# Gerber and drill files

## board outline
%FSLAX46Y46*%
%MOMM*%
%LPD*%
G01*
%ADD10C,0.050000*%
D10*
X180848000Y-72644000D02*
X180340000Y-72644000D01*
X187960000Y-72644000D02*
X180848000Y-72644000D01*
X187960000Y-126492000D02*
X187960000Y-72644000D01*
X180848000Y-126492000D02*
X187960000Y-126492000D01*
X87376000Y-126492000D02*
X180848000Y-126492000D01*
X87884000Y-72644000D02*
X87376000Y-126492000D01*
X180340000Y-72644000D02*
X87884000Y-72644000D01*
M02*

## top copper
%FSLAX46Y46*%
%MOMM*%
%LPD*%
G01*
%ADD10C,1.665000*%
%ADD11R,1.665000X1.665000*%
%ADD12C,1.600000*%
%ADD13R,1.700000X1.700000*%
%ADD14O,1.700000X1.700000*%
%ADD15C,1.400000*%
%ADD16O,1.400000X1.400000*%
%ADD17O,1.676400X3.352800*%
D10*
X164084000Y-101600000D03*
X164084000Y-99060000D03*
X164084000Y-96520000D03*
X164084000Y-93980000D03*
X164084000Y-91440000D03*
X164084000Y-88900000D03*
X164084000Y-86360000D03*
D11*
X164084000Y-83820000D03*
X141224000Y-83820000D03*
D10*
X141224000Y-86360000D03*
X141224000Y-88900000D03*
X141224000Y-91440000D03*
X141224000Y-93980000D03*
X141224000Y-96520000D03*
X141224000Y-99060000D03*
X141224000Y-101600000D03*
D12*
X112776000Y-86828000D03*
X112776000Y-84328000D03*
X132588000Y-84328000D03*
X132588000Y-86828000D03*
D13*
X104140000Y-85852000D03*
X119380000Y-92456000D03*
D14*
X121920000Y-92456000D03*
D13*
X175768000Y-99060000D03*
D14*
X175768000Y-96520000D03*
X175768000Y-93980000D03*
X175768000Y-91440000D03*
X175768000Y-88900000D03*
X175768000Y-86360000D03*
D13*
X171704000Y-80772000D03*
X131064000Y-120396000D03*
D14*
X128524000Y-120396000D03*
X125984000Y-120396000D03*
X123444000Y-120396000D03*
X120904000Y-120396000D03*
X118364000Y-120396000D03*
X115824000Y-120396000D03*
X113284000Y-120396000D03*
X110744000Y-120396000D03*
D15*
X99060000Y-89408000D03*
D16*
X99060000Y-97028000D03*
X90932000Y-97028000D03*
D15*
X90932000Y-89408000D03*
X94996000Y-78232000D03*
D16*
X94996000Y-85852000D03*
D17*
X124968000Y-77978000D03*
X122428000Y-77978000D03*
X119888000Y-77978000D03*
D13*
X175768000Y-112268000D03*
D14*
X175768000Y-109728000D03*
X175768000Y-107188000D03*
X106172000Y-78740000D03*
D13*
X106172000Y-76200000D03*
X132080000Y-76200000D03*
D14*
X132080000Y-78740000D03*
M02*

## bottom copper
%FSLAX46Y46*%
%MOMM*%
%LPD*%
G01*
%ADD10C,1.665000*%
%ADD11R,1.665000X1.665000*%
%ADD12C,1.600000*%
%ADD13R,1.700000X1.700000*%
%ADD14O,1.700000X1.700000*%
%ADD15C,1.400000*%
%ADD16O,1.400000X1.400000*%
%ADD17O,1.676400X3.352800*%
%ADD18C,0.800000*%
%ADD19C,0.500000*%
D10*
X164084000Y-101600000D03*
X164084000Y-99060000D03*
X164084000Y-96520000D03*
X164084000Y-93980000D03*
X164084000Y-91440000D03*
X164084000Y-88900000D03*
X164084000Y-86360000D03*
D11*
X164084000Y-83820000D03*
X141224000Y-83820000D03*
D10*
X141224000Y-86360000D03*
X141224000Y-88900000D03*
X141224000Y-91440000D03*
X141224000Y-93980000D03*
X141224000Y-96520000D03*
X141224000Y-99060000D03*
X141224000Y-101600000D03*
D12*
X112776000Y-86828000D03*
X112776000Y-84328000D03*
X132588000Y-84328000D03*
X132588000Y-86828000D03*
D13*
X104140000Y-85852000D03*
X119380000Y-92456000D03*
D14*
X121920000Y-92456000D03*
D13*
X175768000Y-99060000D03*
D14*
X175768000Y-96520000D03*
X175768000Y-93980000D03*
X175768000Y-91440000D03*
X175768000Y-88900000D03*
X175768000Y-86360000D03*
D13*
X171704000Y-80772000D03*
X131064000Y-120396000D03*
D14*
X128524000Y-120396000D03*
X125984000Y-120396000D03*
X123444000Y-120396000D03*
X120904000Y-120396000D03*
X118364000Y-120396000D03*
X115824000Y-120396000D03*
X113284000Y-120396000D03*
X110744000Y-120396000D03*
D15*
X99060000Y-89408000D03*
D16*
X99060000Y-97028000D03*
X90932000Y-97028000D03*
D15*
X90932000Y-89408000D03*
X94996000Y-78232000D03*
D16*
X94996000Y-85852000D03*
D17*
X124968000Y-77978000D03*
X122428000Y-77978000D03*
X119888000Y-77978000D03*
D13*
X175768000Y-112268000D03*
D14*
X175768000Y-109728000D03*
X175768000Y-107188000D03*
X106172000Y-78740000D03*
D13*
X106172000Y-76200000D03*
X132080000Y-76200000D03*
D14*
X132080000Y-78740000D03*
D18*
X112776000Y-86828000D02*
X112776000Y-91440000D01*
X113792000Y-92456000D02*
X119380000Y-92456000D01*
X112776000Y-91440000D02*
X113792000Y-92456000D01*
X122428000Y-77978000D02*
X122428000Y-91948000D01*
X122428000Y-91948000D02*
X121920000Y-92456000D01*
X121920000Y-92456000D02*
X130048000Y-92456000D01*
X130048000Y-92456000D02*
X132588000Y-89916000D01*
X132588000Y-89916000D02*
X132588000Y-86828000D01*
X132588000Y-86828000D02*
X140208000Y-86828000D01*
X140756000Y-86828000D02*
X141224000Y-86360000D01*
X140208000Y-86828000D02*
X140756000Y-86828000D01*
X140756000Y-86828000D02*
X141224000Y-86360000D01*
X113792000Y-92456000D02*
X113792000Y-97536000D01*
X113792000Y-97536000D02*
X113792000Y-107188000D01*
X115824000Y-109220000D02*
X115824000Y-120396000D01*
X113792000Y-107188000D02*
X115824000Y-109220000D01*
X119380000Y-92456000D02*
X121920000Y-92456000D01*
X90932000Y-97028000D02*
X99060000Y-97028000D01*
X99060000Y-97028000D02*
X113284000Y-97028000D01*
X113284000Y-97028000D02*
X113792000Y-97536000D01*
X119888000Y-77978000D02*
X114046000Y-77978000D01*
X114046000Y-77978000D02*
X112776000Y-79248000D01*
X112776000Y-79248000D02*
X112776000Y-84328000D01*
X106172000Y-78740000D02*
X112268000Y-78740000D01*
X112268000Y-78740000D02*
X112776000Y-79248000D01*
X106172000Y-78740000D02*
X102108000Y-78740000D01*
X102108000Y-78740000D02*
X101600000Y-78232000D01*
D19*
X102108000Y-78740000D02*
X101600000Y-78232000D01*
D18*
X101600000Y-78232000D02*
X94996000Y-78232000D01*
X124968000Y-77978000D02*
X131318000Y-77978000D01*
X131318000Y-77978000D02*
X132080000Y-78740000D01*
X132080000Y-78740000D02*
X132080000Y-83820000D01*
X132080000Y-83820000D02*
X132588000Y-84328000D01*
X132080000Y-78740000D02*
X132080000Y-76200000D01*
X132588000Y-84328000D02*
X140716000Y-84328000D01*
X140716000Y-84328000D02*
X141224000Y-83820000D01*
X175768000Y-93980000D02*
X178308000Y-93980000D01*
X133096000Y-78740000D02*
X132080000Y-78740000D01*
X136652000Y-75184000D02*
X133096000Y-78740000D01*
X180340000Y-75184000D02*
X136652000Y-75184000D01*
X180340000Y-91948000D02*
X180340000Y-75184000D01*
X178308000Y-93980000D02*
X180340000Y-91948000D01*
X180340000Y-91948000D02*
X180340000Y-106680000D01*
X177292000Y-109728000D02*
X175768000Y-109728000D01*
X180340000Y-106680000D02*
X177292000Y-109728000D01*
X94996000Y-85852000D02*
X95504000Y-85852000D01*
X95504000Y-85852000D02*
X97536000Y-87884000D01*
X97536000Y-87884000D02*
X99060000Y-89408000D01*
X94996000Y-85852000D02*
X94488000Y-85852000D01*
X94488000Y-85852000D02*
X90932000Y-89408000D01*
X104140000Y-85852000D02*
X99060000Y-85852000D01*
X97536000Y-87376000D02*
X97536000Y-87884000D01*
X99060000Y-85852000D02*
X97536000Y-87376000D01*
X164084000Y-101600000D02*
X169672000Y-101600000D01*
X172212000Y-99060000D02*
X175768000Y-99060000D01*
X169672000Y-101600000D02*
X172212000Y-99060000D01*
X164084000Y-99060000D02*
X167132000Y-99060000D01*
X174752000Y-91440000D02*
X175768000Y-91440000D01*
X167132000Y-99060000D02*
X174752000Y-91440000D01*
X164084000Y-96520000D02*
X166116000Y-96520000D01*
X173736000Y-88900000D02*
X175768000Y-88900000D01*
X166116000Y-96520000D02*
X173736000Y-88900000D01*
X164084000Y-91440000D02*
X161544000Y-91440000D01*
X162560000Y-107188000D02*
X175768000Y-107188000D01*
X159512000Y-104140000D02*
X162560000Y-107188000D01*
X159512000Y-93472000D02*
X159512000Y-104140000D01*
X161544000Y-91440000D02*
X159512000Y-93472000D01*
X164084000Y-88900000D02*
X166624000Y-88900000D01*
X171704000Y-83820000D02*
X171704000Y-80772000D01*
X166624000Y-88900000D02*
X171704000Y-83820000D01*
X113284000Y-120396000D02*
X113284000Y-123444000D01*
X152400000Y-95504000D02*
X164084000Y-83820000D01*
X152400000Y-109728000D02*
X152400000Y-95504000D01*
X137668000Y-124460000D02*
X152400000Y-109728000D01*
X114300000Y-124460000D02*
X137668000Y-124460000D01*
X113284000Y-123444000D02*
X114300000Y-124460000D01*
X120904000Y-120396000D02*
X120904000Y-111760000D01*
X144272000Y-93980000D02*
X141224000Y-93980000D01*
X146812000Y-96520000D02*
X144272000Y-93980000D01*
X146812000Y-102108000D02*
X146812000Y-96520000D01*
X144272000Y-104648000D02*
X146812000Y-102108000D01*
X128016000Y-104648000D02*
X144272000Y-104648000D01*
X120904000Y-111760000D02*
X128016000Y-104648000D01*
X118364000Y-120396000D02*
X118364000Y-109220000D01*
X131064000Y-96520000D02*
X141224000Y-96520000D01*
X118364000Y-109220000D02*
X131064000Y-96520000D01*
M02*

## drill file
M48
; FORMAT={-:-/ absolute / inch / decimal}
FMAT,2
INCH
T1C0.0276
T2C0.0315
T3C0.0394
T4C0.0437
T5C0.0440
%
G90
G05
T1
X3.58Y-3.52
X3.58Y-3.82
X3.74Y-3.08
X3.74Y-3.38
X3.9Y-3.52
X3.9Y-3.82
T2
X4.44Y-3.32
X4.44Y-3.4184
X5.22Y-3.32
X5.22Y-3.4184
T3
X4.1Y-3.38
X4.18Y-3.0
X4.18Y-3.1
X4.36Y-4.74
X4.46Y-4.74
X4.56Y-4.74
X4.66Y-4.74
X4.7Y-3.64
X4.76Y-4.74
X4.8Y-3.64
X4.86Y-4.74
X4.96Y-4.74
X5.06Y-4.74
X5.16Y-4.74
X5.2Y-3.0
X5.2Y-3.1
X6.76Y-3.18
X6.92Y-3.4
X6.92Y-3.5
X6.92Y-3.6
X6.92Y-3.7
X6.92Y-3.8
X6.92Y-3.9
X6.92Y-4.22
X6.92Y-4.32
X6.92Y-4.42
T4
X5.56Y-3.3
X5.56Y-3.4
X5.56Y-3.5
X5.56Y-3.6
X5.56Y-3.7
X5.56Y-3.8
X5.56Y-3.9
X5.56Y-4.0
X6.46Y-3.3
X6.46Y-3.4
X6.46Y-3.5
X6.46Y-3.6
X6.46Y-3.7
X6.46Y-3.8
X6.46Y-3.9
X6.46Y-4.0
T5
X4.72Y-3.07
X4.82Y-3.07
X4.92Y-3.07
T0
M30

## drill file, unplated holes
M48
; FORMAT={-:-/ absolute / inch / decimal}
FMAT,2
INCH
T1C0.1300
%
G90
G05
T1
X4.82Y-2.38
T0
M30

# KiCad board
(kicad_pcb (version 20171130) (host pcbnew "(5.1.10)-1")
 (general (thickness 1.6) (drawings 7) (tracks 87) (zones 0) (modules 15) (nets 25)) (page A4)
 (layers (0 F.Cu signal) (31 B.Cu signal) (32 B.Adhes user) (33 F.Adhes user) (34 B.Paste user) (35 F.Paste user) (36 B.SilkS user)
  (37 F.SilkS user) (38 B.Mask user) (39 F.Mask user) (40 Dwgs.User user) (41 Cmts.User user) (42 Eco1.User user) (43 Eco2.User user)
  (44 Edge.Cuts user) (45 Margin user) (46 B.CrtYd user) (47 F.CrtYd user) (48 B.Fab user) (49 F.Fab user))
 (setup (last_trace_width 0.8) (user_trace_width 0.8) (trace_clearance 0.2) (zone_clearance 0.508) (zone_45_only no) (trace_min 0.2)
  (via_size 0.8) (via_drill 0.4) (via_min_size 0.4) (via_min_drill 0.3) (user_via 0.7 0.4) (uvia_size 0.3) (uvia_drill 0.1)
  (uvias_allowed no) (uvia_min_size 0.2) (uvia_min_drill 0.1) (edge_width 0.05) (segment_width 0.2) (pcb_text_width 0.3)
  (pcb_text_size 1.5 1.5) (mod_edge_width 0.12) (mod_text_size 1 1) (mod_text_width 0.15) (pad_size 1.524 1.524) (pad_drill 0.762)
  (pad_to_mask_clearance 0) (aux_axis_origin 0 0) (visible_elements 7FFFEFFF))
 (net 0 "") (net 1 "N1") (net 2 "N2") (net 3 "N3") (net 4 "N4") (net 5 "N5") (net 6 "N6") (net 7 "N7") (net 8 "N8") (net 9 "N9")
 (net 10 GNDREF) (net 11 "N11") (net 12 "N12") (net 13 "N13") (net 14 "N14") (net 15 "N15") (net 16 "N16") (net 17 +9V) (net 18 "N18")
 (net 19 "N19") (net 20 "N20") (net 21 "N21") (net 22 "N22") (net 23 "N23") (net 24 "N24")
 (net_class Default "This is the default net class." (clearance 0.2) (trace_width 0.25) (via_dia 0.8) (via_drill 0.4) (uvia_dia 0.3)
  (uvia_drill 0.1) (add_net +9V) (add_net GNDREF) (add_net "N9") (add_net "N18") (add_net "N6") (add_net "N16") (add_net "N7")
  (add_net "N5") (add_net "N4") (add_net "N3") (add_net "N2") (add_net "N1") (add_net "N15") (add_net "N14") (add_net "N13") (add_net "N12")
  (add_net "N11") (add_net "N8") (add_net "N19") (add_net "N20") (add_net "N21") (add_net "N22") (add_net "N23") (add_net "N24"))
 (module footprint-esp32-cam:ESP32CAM (layer F.Cu) (at 141.224 101.6)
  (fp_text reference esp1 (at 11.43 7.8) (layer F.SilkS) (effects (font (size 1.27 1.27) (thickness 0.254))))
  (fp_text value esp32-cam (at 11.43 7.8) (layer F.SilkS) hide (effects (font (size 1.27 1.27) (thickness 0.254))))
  (pad 16 thru_hole circle (at 22.86 0) (size 1.665 1.665) (drill 1.11) (layers *.Cu *.Mask) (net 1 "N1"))
  (pad 15 thru_hole circle (at 22.86 -2.54) (size 1.665 1.665) (drill 1.11) (layers *.Cu *.Mask) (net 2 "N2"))
  (pad 14 thru_hole circle (at 22.86 -5.08) (size 1.665 1.665) (drill 1.11) (layers *.Cu *.Mask) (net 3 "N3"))
  (pad 13 thru_hole circle (at 22.86 -7.62) (size 1.665 1.665) (drill 1.11) (layers *.Cu *.Mask) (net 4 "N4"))
  (pad 12 thru_hole circle (at 22.86 -10.16) (size 1.665 1.665) (drill 1.11) (layers *.Cu *.Mask) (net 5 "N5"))
  (pad 11 thru_hole circle (at 22.86 -12.7) (size 1.665 1.665) (drill 1.11) (layers *.Cu *.Mask) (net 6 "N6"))
  (pad 10 thru_hole circle (at 22.86 -15.24) (size 1.665 1.665) (drill 1.11) (layers *.Cu *.Mask) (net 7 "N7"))
  (pad 9 thru_hole rect (at 22.86 -17.78) (size 1.665 1.665) (drill 1.11) (layers *.Cu *.Mask) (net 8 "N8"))
  (pad 8 thru_hole rect (at 0 -17.78) (size 1.665 1.665) (drill 1.11) (layers *.Cu *.Mask) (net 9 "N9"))
  (pad 7 thru_hole circle (at 0 -15.24) (size 1.665 1.665) (drill 1.11) (layers *.Cu *.Mask) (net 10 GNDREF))
  (pad 6 thru_hole circle (at 0 -12.7) (size 1.665 1.665) (drill 1.11) (layers *.Cu *.Mask) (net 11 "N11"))
  (pad 5 thru_hole circle (at 0 -10.16) (size 1.665 1.665) (drill 1.11) (layers *.Cu *.Mask) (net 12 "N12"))
  (pad 4 thru_hole circle (at 0 -7.62) (size 1.665 1.665) (drill 1.11) (layers *.Cu *.Mask) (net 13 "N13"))
  (pad 3 thru_hole circle (at 0 -5.08) (size 1.665 1.665) (drill 1.11) (layers *.Cu *.Mask) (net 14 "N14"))
  (pad 2 thru_hole circle (at 0 -2.54) (size 1.665 1.665) (drill 1.11) (layers *.Cu *.Mask) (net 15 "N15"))
  (pad 1 thru_hole circle (at 0 0) (size 1.665 1.665) (drill 1.11) (layers *.Cu *.Mask) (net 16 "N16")))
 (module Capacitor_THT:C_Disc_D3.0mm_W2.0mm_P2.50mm (layer F.Cu) (at 112.776 84.328 270)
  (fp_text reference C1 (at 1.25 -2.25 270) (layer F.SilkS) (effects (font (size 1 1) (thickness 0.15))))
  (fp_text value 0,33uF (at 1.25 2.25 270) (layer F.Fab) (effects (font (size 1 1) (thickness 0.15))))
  (pad 2 thru_hole circle (at 2.5 0 270) (size 1.6 1.6) (drill 0.8) (layers *.Cu *.Mask) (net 10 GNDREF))
  (pad 1 thru_hole circle (at 0 0 270) (size 1.6 1.6) (drill 0.8) (layers *.Cu *.Mask) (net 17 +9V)))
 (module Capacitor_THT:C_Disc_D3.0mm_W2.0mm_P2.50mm (layer F.Cu) (at 132.588 84.328 270)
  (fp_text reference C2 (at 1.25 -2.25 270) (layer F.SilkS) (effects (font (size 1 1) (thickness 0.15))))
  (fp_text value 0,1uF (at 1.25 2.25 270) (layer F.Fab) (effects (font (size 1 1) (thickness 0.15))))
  (pad 1 thru_hole circle (at 0 0 270) (size 1.6 1.6) (drill 0.8) (layers *.Cu *.Mask) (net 9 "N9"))
  (pad 2 thru_hole circle (at 2.5 0 270) (size 1.6 1.6) (drill 0.8) (layers *.Cu *.Mask) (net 10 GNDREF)))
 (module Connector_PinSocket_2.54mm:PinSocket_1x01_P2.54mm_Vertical (layer F.Cu) (at 104.14 85.852)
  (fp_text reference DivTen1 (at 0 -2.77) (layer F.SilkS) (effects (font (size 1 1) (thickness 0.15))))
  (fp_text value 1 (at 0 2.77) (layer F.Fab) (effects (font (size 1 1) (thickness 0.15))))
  (pad 1 thru_hole rect (at 0 0) (size 1.7 1.7) (drill 1) (layers *.Cu *.Mask) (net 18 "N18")))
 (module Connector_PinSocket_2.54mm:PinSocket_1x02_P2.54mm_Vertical (layer F.Cu) (at 119.38 92.456 90)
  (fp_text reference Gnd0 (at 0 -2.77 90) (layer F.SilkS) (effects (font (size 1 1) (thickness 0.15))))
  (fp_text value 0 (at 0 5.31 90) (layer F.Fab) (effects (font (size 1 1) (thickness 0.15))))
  (pad 1 thru_hole rect (at 0 0 90) (size 1.7 1.7) (drill 1) (layers *.Cu *.Mask) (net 10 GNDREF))
  (pad 2 thru_hole oval (at 0 2.54 90) (size 1.7 1.7) (drill 1) (layers *.Cu *.Mask) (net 10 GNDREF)))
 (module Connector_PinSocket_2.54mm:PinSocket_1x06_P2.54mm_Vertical (layer F.Cu) (at 175.768 99.06 180)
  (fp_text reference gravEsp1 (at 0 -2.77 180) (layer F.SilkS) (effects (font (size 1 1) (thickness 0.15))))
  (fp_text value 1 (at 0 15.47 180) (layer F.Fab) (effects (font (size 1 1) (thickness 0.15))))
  (pad 1 thru_hole rect (at 0 0 180) (size 1.7 1.7) (drill 1) (layers *.Cu *.Mask) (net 1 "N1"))
  (pad 2 thru_hole oval (at 0 2.54 180) (size 1.7 1.7) (drill 1) (layers *.Cu *.Mask) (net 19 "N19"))
  (pad 3 thru_hole oval (at 0 5.08 180) (size 1.7 1.7) (drill 1) (layers *.Cu *.Mask) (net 9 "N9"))
  (pad 4 thru_hole oval (at 0 7.62 180) (size 1.7 1.7) (drill 1) (layers *.Cu *.Mask) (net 2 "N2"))
  (pad 5 thru_hole oval (at 0 10.16 180) (size 1.7 1.7) (drill 1) (layers *.Cu *.Mask) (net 3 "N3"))
  (pad 6 thru_hole oval (at 0 12.7 180) (size 1.7 1.7) (drill 1) (layers *.Cu *.Mask) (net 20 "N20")))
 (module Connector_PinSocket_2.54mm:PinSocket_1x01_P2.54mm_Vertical (layer F.Cu) (at 171.704 80.772)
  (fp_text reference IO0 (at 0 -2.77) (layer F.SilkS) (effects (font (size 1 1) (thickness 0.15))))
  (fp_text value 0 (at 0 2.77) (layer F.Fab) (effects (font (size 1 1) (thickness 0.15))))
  (pad 1 thru_hole rect (at 0 0) (size 1.7 1.7) (drill 1) (layers *.Cu *.Mask) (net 6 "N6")))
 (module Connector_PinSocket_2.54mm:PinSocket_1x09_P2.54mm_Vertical (layer F.Cu) (at 131.064 120.396 270)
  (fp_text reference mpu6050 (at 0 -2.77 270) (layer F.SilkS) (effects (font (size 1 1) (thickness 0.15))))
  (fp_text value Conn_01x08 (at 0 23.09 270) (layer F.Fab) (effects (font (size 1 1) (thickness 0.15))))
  (pad 1 thru_hole rect (at 0 0 270) (size 1.7 1.7) (drill 1) (layers *.Cu *.Mask) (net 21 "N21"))
  (pad 2 thru_hole oval (at 0 2.54 270) (size 1.7 1.7) (drill 1) (layers *.Cu *.Mask) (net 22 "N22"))
  (pad 3 thru_hole oval (at 0 5.08 270) (size 1.7 1.7) (drill 1) (layers *.Cu *.Mask) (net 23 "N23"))
  (pad 4 thru_hole oval (at 0 7.62 270) (size 1.7 1.7) (drill 1) (layers *.Cu *.Mask) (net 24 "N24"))
  (pad 5 thru_hole oval (at 0 10.16 270) (size 1.7 1.7) (drill 1) (layers *.Cu *.Mask) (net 13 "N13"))
  (pad 6 thru_hole oval (at 0 12.7 270) (size 1.7 1.7) (drill 1) (layers *.Cu *.Mask) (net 14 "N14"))
  (pad 7 thru_hole oval (at 0 15.24 270) (size 1.7 1.7) (drill 1) (layers *.Cu *.Mask) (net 10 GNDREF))
  (pad 8 thru_hole oval (at 0 17.78 270) (size 1.7 1.7) (drill 1) (layers *.Cu *.Mask) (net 8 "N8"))
  (pad 9 thru_hole oval (at 0 20.32 270) (size 1.7 1.7) (drill 1) (layers *.Cu *.Mask)))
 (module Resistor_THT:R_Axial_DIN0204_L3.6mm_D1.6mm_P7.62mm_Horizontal (layer F.Cu) (at 99.06 89.408 270)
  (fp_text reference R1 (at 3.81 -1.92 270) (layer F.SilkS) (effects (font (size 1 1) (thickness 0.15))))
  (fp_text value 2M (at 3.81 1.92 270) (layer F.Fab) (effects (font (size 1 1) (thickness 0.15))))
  (pad 1 thru_hole circle (at 0 0 270) (size 1.4 1.4) (drill 0.7) (layers *.Cu *.Mask) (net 18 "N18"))
  (pad 2 thru_hole oval (at 7.62 0 270) (size 1.4 1.4) (drill 0.7) (layers *.Cu *.Mask) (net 10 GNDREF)))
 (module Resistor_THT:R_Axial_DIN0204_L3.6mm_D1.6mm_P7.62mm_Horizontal (layer F.Cu) (at 90.932 89.408 270)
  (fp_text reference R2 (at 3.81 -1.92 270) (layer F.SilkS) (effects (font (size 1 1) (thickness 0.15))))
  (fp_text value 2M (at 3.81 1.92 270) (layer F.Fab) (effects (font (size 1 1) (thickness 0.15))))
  (pad 2 thru_hole oval (at 7.62 0 270) (size 1.4 1.4) (drill 0.7) (layers *.Cu *.Mask) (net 10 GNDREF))
  (pad 1 thru_hole circle (at 0 0 270) (size 1.4 1.4) (drill 0.7) (layers *.Cu *.Mask) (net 18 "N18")))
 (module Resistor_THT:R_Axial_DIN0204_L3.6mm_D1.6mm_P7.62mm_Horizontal (layer F.Cu) (at 94.996 78.232 270)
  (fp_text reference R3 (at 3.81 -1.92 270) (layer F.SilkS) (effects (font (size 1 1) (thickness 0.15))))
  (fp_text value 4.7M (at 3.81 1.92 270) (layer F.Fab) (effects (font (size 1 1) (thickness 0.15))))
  (pad 1 thru_hole circle (at 0 0 270) (size 1.4 1.4) (drill 0.7) (layers *.Cu *.Mask) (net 17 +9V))
  (pad 2 thru_hole oval (at 7.62 0 270) (size 1.4 1.4) (drill 0.7) (layers *.Cu *.Mask) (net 18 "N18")))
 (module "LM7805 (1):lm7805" (layer F.Cu) (at 122.428 71.628)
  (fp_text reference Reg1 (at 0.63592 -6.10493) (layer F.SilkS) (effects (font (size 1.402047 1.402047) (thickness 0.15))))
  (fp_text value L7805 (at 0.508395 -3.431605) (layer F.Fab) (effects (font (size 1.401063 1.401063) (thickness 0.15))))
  (pad None np_thru_hole circle (at 0 -11.176) (size 3.302 3.302) (drill 3.302) (layers *.Cu *.Mask))
  (pad 3 thru_hole oval (at 2.54 6.35) (size 1.6764 3.3528) (drill 1.1176) (layers *.Cu *.Mask) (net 9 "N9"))
  (pad 2 thru_hole oval (at 0 6.35) (size 1.6764 3.3528) (drill 1.1176) (layers *.Cu *.Mask) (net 10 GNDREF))
  (pad 1 thru_hole oval (at -2.54 6.35) (size 1.6764 3.3528) (drill 1.1176) (layers *.Cu *.Mask) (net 17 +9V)))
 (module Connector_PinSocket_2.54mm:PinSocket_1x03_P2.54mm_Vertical (layer F.Cu) (at 175.768 112.268 180)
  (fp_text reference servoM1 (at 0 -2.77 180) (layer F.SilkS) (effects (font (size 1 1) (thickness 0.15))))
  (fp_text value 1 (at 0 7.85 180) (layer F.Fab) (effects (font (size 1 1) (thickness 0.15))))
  (pad 1 thru_hole rect (at 0 0 180) (size 1.7 1.7) (drill 1) (layers *.Cu *.Mask) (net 16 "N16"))
  (pad 2 thru_hole oval (at 0 2.54 180) (size 1.7 1.7) (drill 1) (layers *.Cu *.Mask) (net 9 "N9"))
  (pad 3 thru_hole oval (at 0 5.08 180) (size 1.7 1.7) (drill 1) (layers *.Cu *.Mask) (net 5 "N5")))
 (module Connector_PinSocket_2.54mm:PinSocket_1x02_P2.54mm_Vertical (layer F.Cu) (at 106.172 76.2)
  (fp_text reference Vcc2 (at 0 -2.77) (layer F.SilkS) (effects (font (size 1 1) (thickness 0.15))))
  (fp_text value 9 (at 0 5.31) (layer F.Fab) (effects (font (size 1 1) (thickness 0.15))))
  (pad 2 thru_hole oval (at 0 2.54) (size 1.7 1.7) (drill 1) (layers *.Cu *.Mask) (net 17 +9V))
  (pad 1 thru_hole rect (at 0 0) (size 1.7 1.7) (drill 1) (layers *.Cu *.Mask) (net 17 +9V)))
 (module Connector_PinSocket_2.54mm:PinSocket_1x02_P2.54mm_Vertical (layer F.Cu) (at 132.08 76.2)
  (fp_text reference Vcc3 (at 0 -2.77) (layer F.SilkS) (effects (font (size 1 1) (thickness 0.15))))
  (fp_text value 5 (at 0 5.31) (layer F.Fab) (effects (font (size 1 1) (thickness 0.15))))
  (pad 1 thru_hole rect (at 0 0) (size 1.7 1.7) (drill 1) (layers *.Cu *.Mask) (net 9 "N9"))
  (pad 2 thru_hole oval (at 0 2.54) (size 1.7 1.7) (drill 1) (layers *.Cu *.Mask) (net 9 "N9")))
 (gr_line (start 180.848 72.644) (end 180.34 72.644) (angle 90) (layer Edge.Cuts) (width 0.05))
 (gr_line (start 187.96 72.644) (end 180.848 72.644) (angle 90) (layer Edge.Cuts) (width 0.05))
 (gr_line (start 187.96 126.492) (end 187.96 72.644) (angle 90) (layer Edge.Cuts) (width 0.05))
 (gr_line (start 180.848 126.492) (end 187.96 126.492) (angle 90) (layer Edge.Cuts) (width 0.05))
 (gr_line (start 87.376 126.492) (end 180.848 126.492) (angle 90) (layer Edge.Cuts) (width 0.05))
 (gr_line (start 87.884 72.644) (end 87.376 126.492) (angle 90) (layer Edge.Cuts) (width 0.05))
 (gr_line (start 180.34 72.644) (end 87.884 72.644) (angle 90) (layer Edge.Cuts) (width 0.05))
 (segment (start 112.776 86.828) (end 112.776 91.44) (width 0.8) (layer B.Cu) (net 10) (status 400000))
 (segment (start 113.792 92.456) (end 119.38 92.456) (width 0.8) (layer B.Cu) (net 10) (status 800000))
 (segment (start 112.776 91.44) (end 113.792 92.456) (width 0.8) (layer B.Cu) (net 10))
 (segment (start 122.428 77.978) (end 122.428 91.948) (width 0.8) (layer B.Cu) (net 10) (status C00000))
 (segment (start 122.428 91.948) (end 121.92 92.456) (width 0.8) (layer B.Cu) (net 10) (status C00000))
 (segment (start 121.92 92.456) (end 130.048 92.456) (width 0.8) (layer B.Cu) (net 10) (status 400000))
 (segment (start 130.048 92.456) (end 132.588 89.916) (width 0.8) (layer B.Cu) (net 10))
 (segment (start 132.588 89.916) (end 132.588 86.828) (width 0.8) (layer B.Cu) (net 10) (status 800000))
 (segment (start 132.588 86.828) (end 140.208 86.828) (width 0.8) (layer B.Cu) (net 10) (status 400000))
 (segment (start 140.756 86.828) (end 141.224 86.36) (width 0.8) (layer B.Cu) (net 10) (status C00000))
 (segment (start 140.208 86.828) (end 140.756 86.828) (width 0.8) (layer B.Cu) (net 10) (status 800000))
 (segment (start 140.756 86.828) (end 141.224 86.36) (width 0.8) (layer B.Cu) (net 10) (status C00000))
 (segment (start 113.792 92.456) (end 113.792 97.536) (width 0.8) (layer B.Cu) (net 10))
 (segment (start 113.792 97.536) (end 113.792 107.188) (width 0.8) (layer B.Cu) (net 10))
 (segment (start 115.824 109.22) (end 115.824 120.396) (width 0.8) (layer B.Cu) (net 10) (status 800000))
 (segment (start 113.792 107.188) (end 115.824 109.22) (width 0.8) (layer B.Cu) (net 10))
 (segment (start 119.38 92.456) (end 121.92 92.456) (width 0.8) (layer B.Cu) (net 10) (status C00000))
 (segment (start 90.932 97.028) (end 99.06 97.028) (width 0.8) (layer B.Cu) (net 10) (status C00000))
 (segment (start 99.06 97.028) (end 113.284 97.028) (width 0.8) (layer B.Cu) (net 10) (status 400000))
 (segment (start 113.284 97.028) (end 113.792 97.536) (width 0.8) (layer B.Cu) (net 10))
 (segment (start 119.888 77.978) (end 114.046 77.978) (width 0.8) (layer B.Cu) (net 17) (status 400000))
 (segment (start 114.046 77.978) (end 112.776 79.248) (width 0.8) (layer B.Cu) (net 17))
 (segment (start 112.776 79.248) (end 112.776 84.328) (width 0.8) (layer B.Cu) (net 17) (status 800000))
 (segment (start 106.172 78.74) (end 112.268 78.74) (width 0.8) (layer B.Cu) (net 17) (status 400000))
 (segment (start 112.268 78.74) (end 112.776 79.248) (width 0.8) (layer B.Cu) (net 17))
 (segment (start 106.172 78.74) (end 102.108 78.74) (width 0.8) (layer B.Cu) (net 17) (status 400000))
 (segment (start 102.108 78.74) (end 101.6 78.232) (width 0.8) (layer B.Cu) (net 17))
 (segment (start 102.108 78.74) (end 101.6 78.232) (width 0.5) (layer B.Cu) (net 17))
 (segment (start 101.6 78.232) (end 94.996 78.232) (width 0.8) (layer B.Cu) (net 17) (status 800000))
 (segment (start 124.968 77.978) (end 131.318 77.978) (width 0.8) (layer B.Cu) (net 9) (status 400000))
 (segment (start 131.318 77.978) (end 132.08 78.74) (width 0.8) (layer B.Cu) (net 9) (status 800000))
 (segment (start 132.08 78.74) (end 132.08 83.82) (width 0.8) (layer B.Cu) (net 9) (status C00000))
 (segment (start 132.08 83.82) (end 132.588 84.328) (width 0.8) (layer B.Cu) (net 9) (status C00000))
 (segment (start 132.08 78.74) (end 132.08 76.2) (width 0.8) (layer B.Cu) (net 9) (status C00000))
 (segment (start 140.716 84.328) (end 141.224 83.82) (width 0.8) (layer B.Cu) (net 9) (status C00000))
 (segment (start 175.768 93.98) (end 178.308 93.98) (width 0.8) (layer B.Cu) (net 9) (status 400000))
 (segment (start 133.096 78.74) (end 132.08 78.74) (width 0.8) (layer B.Cu) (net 9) (status 800000))
 (segment (start 136.652 75.184) (end 133.096 78.74) (width 0.8) (layer B.Cu) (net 9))
 (segment (start 180.34 75.184) (end 136.652 75.184) (width 0.8) (layer B.Cu) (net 9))
 (segment (start 180.34 91.948) (end 180.34 75.184) (width 0.8) (layer B.Cu) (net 9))
 (segment (start 178.308 93.98) (end 180.34 91.948) (width 0.8) (layer B.Cu) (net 9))
 (segment (start 180.34 91.948) (end 180.34 106.68) (width 0.8) (layer B.Cu) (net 9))
 (segment (start 177.292 109.728) (end 175.768 109.728) (width 0.8) (layer B.Cu) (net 9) (status 800000))
 (segment (start 180.34 106.68) (end 177.292 109.728) (width 0.8) (layer B.Cu) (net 9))
 (segment (start 132.588 84.328) (end 140.716 84.328) (width 0.8) (layer B.Cu) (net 9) (status C00000))
 (segment (start 140.716 84.328) (end 141.224 83.82) (width 0.8) (layer B.Cu) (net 9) (status C00000))
 (segment (start 94.996 85.852) (end 95.504 85.852) (width 0.8) (layer B.Cu) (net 18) (status C00000))
 (segment (start 95.504 85.852) (end 97.536 87.884) (width 0.8) (layer B.Cu) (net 18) (status 400000))
 (segment (start 97.536 87.884) (end 99.06 89.408) (width 0.8) (layer B.Cu) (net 18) (status 800000))
 (segment (start 94.996 85.852) (end 94.488 85.852) (width 0.8) (layer B.Cu) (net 18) (status C00000))
 (segment (start 94.488 85.852) (end 90.932 89.408) (width 0.8) (layer B.Cu) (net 18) (status C00000))
 (segment (start 104.14 85.852) (end 99.06 85.852) (width 0.8) (layer B.Cu) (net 18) (status 400000))
 (segment (start 97.536 87.376) (end 97.536 87.884) (width 0.8) (layer B.Cu) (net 18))
 (segment (start 99.06 85.852) (end 97.536 87.376) (width 0.8) (layer B.Cu) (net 18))
 (segment (start 164.084 101.6) (end 169.672 101.6) (width 0.8) (layer B.Cu) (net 1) (status 400000))
 (segment (start 172.212 99.06) (end 175.768 99.06) (width 0.8) (layer B.Cu) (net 1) (status 800000))
 (segment (start 169.672 101.6) (end 172.212 99.06) (width 0.8) (layer B.Cu) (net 1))
 (segment (start 164.084 99.06) (end 167.132 99.06) (width 0.8) (layer B.Cu) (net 2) (status 400000))
 (segment (start 174.752 91.44) (end 175.768 91.44) (width 0.8) (layer B.Cu) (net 2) (status 800000))
 (segment (start 167.132 99.06) (end 174.752 91.44) (width 0.8) (layer B.Cu) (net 2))
 (segment (start 164.084 96.52) (end 166.116 96.52) (width 0.8) (layer B.Cu) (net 3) (status 400000))
 (segment (start 173.736 88.9) (end 175.768 88.9) (width 0.8) (layer B.Cu) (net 3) (status 800000))
 (segment (start 166.116 96.52) (end 173.736 88.9) (width 0.8) (layer B.Cu) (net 3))
 (segment (start 164.084 91.44) (end 161.544 91.44) (width 0.8) (layer B.Cu) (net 5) (status 400000))
 (segment (start 162.56 107.188) (end 175.768 107.188) (width 0.8) (layer B.Cu) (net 5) (status 800000))
 (segment (start 159.512 104.14) (end 162.56 107.188) (width 0.8) (layer B.Cu) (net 5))
 (segment (start 159.512 93.472) (end 159.512 104.14) (width 0.8) (layer B.Cu) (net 5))
 (segment (start 161.544 91.44) (end 159.512 93.472) (width 0.8) (layer B.Cu) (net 5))
 (segment (start 164.084 88.9) (end 166.624 88.9) (width 0.8) (layer B.Cu) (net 6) (status 400000))
 (segment (start 171.704 83.82) (end 171.704 80.772) (width 0.8) (layer B.Cu) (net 6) (status 800000))
 (segment (start 166.624 88.9) (end 171.704 83.82) (width 0.8) (layer B.Cu) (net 6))
 (segment (start 113.284 120.396) (end 113.284 123.444) (width 0.8) (layer B.Cu) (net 8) (status 400000))
 (segment (start 152.4 95.504) (end 164.084 83.82) (width 0.8) (layer B.Cu) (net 8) (status 800000))
 (segment (start 152.4 109.728) (end 152.4 95.504) (width 0.8) (layer B.Cu) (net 8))
 (segment (start 137.668 124.46) (end 152.4 109.728) (width 0.8) (layer B.Cu) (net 8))
 (segment (start 114.3 124.46) (end 137.668 124.46) (width 0.8) (layer B.Cu) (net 8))
 (segment (start 113.284 123.444) (end 114.3 124.46) (width 0.8) (layer B.Cu) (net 8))
 (segment (start 120.904 120.396) (end 120.904 111.76) (width 0.8) (layer B.Cu) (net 13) (status 400000))
 (segment (start 144.272 93.98) (end 141.224 93.98) (width 0.8) (layer B.Cu) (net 13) (status 800000))
 (segment (start 146.812 96.52) (end 144.272 93.98) (width 0.8) (layer B.Cu) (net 13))
 (segment (start 146.812 102.108) (end 146.812 96.52) (width 0.8) (layer B.Cu) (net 13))
 (segment (start 144.272 104.648) (end 146.812 102.108) (width 0.8) (layer B.Cu) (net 13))
 (segment (start 128.016 104.648) (end 144.272 104.648) (width 0.8) (layer B.Cu) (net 13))
 (segment (start 120.904 111.76) (end 128.016 104.648) (width 0.8) (layer B.Cu) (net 13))
 (segment (start 118.364 120.396) (end 118.364 109.22) (width 0.8) (layer B.Cu) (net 14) (status 400000))
 (segment (start 131.064 96.52) (end 141.224 96.52) (width 0.8) (layer B.Cu) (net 14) (status 800000))
 (segment (start 118.364 109.22) (end 131.064 96.52) (width 0.8) (layer B.Cu) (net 14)))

